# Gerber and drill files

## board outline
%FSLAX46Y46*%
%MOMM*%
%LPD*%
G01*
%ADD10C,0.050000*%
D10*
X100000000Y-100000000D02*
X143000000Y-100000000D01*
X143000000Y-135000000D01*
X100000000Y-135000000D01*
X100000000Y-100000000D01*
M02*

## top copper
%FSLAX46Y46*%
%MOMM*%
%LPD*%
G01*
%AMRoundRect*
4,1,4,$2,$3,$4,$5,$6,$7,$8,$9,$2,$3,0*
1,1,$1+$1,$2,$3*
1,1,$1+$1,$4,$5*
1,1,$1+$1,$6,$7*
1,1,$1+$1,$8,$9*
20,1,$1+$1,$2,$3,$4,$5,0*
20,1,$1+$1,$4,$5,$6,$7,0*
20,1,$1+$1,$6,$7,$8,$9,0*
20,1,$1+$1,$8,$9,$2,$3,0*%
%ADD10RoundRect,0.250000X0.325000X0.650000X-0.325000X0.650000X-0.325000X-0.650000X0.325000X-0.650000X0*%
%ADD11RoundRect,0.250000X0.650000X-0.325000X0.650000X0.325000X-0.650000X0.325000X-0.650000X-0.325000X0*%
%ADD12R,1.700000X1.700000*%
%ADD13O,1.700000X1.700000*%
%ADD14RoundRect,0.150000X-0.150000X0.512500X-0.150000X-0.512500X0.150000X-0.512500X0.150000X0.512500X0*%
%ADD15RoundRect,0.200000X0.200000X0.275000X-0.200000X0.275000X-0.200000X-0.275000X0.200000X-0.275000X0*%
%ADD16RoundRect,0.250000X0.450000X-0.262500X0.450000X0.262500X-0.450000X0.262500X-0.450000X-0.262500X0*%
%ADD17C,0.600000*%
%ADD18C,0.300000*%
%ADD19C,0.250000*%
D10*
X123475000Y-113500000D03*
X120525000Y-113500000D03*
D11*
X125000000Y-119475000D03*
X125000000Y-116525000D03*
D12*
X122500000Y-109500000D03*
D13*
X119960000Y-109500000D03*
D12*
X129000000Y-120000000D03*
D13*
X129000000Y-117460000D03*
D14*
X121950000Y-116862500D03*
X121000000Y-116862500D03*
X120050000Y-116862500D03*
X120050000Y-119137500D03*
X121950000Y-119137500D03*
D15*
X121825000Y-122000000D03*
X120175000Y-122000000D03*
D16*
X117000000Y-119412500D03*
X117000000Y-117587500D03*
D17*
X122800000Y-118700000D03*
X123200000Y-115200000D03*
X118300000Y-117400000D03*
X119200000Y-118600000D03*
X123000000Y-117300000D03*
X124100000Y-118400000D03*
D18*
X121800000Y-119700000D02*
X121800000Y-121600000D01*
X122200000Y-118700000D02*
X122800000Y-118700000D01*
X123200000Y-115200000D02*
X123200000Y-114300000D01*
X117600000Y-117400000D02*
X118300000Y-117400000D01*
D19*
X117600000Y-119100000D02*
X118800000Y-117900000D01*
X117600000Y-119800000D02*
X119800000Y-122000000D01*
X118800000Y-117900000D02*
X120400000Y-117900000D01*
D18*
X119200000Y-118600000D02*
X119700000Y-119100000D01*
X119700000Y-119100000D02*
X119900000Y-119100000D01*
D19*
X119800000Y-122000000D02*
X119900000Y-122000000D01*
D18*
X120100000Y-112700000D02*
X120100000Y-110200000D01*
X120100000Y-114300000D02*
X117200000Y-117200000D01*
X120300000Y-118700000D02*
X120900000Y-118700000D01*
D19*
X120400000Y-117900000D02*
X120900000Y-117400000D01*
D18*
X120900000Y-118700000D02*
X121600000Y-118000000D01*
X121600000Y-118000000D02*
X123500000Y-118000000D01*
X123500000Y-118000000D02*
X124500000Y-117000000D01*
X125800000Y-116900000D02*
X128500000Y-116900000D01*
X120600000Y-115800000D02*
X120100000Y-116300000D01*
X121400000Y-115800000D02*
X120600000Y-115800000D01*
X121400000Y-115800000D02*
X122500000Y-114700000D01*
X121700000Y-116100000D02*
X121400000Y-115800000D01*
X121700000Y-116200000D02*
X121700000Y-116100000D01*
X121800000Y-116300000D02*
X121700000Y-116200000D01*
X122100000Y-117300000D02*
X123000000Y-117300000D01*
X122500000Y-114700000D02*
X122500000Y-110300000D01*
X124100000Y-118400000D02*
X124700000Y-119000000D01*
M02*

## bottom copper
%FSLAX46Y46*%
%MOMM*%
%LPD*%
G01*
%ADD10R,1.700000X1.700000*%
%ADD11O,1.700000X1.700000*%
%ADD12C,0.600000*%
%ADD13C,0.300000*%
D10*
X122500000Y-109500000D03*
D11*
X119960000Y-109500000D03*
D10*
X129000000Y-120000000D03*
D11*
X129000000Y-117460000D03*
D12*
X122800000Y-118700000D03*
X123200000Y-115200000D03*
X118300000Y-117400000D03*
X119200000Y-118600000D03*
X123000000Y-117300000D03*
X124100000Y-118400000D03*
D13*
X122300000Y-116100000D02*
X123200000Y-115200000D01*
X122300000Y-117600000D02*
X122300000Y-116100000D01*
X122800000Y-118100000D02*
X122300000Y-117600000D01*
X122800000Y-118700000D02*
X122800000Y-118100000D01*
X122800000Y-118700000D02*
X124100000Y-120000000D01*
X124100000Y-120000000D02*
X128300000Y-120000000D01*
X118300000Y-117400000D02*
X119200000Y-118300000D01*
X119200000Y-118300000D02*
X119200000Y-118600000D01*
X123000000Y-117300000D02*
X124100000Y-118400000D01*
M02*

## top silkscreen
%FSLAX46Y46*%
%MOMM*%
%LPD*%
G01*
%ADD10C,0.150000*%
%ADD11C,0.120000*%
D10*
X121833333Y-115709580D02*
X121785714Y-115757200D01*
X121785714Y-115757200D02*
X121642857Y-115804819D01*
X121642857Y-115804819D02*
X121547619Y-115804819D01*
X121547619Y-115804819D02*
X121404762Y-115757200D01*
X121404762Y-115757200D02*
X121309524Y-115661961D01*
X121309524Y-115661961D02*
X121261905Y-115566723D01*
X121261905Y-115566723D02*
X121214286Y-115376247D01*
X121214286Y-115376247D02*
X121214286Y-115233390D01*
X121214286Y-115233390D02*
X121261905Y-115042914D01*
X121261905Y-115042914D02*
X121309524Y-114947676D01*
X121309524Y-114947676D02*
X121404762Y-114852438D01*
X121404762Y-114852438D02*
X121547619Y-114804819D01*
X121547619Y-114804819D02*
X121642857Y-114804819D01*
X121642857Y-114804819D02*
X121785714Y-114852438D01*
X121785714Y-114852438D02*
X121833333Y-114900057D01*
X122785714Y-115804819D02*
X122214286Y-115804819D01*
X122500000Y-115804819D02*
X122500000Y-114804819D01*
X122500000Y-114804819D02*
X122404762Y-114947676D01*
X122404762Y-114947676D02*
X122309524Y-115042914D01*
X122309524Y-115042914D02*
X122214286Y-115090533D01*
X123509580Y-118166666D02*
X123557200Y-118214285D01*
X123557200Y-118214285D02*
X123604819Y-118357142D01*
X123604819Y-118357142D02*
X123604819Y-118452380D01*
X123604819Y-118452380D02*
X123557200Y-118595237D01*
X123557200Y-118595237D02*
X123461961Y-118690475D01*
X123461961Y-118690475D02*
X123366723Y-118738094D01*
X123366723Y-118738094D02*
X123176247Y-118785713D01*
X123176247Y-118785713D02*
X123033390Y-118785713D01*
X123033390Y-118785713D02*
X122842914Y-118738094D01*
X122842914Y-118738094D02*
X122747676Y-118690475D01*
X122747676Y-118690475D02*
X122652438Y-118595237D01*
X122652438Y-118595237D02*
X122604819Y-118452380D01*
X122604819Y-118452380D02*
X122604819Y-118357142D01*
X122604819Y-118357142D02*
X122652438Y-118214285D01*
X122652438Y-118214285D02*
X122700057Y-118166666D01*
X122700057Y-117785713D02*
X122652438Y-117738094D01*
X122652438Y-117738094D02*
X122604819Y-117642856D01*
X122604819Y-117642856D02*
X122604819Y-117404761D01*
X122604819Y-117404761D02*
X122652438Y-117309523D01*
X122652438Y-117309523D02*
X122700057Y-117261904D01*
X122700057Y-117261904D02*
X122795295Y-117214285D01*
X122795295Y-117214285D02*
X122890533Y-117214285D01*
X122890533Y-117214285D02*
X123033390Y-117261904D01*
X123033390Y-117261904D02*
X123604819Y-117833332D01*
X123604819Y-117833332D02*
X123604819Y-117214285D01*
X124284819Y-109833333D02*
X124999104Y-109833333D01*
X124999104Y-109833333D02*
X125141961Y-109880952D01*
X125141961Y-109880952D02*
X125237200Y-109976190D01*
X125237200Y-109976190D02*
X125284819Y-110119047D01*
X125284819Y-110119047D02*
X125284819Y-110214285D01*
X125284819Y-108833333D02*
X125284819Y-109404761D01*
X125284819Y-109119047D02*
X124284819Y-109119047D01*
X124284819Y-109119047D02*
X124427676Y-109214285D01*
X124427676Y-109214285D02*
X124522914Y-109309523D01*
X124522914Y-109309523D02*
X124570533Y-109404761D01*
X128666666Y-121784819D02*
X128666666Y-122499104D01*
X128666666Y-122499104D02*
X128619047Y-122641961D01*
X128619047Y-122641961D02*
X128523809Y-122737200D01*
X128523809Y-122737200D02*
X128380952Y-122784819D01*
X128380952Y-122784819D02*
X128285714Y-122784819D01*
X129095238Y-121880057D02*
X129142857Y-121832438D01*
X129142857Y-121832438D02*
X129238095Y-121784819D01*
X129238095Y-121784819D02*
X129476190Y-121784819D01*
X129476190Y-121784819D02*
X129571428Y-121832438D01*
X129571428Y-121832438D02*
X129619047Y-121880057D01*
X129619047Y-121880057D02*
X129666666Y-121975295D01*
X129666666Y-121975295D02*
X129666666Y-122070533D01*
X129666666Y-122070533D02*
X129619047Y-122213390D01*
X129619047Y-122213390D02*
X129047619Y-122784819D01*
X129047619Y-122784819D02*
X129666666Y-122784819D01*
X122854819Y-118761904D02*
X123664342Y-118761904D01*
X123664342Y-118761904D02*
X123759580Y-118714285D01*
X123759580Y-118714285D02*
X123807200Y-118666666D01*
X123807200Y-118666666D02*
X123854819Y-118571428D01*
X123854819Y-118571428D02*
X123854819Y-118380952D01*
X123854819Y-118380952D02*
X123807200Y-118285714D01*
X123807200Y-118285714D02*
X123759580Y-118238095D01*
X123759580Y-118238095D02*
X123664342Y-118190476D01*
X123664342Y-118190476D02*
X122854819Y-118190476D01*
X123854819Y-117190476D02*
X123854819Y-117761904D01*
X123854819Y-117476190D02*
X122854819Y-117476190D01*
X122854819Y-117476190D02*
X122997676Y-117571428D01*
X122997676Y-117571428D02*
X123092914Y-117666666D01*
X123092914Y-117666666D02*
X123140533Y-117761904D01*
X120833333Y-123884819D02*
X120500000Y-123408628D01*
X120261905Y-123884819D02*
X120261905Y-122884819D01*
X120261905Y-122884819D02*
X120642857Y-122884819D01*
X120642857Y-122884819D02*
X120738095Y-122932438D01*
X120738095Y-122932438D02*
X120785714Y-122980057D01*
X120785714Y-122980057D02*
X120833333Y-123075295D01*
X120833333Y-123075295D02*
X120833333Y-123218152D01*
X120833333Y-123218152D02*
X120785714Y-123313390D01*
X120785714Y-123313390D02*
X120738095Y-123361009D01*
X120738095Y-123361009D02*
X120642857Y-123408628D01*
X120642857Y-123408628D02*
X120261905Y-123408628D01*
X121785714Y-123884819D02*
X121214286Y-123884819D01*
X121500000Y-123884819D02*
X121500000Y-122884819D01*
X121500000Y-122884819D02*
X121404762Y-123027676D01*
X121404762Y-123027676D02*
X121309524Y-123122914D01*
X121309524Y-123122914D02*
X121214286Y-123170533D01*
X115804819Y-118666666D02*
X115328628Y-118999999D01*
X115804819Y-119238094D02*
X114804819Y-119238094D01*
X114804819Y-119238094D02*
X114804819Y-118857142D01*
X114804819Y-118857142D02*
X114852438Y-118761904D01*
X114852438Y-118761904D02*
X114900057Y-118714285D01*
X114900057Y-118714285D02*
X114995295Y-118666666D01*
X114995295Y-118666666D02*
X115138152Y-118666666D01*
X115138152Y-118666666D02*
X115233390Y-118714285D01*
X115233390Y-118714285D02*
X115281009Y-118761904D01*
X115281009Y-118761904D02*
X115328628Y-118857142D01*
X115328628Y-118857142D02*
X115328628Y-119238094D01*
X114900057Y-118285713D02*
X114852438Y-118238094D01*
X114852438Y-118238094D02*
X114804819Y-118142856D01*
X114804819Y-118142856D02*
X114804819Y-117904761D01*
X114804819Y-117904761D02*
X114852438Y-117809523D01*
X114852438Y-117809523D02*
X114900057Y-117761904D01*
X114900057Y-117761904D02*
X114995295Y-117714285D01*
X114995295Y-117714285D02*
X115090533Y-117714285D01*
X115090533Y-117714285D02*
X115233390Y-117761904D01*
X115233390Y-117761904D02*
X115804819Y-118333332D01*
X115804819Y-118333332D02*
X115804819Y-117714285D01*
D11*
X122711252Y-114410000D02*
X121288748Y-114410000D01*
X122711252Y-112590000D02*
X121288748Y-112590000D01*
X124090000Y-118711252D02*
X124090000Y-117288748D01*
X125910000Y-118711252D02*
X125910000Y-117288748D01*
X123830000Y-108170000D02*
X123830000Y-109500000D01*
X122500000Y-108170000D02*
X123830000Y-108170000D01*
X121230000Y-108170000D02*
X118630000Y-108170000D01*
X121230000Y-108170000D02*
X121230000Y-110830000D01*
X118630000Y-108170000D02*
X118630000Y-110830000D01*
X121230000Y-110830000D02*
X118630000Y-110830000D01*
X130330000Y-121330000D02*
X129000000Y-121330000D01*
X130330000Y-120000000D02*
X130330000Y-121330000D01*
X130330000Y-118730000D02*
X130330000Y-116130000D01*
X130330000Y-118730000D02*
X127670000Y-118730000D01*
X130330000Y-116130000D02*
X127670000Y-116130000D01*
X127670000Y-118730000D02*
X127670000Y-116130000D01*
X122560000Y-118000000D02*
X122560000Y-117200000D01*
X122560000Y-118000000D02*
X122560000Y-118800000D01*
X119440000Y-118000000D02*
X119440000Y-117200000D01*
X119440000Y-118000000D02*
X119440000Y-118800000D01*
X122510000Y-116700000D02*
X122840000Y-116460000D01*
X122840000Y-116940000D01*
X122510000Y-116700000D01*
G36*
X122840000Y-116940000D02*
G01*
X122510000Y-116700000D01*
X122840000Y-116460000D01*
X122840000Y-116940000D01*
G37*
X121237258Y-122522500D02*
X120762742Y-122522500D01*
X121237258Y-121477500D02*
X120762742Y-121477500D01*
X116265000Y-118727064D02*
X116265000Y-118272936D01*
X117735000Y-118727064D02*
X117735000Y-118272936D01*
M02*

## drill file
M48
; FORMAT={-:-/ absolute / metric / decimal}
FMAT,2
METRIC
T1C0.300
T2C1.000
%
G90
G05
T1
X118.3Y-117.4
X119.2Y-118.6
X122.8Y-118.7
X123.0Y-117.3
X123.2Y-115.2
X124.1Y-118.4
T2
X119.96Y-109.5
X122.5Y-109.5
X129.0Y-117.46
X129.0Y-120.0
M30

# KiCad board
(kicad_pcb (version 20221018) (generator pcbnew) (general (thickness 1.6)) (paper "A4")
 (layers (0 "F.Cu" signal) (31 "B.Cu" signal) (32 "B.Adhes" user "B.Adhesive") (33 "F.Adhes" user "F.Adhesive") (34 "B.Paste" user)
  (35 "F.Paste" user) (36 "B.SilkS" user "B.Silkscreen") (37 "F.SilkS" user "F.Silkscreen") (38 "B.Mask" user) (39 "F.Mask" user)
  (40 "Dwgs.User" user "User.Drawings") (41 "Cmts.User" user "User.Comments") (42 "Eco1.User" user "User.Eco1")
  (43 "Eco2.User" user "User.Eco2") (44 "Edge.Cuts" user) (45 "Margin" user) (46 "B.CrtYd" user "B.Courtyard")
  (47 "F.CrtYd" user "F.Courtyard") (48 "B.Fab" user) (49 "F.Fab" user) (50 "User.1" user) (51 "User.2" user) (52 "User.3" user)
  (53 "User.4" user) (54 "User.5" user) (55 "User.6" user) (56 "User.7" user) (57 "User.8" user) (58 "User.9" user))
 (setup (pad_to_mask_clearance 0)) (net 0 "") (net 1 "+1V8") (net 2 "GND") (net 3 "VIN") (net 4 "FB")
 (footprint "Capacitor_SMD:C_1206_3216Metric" (layer "F.Cu") (at 122 113.5 180)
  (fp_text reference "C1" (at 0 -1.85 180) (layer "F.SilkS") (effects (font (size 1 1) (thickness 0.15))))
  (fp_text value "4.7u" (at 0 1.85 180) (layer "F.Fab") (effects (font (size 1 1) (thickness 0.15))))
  (fp_line (start -0.711252 -0.91) (end 0.711252 -0.91) (stroke (width 0.12) (type solid)) (layer "F.SilkS"))
  (fp_line (start -0.711252 0.91) (end 0.711252 0.91) (stroke (width 0.12) (type solid)) (layer "F.SilkS"))
  (pad "1" smd roundrect (at -1.475 0 180) (size 1.15 1.8) (layers "F.Cu" "F.Paste" "F.Mask") (roundrect_rratio 0.217391) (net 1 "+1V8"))
  (pad "2" smd roundrect (at 1.475 0 180) (size 1.15 1.8) (layers "F.Cu" "F.Paste" "F.Mask") (roundrect_rratio 0.217391) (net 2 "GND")))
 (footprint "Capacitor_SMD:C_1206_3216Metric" (layer "F.Cu") (at 125 118 90)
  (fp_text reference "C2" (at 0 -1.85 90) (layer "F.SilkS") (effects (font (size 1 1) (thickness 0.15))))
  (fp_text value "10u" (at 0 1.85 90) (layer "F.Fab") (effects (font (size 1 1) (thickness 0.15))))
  (fp_line (start -0.711252 -0.91) (end 0.711252 -0.91) (stroke (width 0.12) (type solid)) (layer "F.SilkS"))
  (fp_line (start -0.711252 0.91) (end 0.711252 0.91) (stroke (width 0.12) (type solid)) (layer "F.SilkS"))
  (pad "1" smd roundrect (at -1.475 0 90) (size 1.15 1.8) (layers "F.Cu" "F.Paste" "F.Mask") (roundrect_rratio 0.217391) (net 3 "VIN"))
  (pad "2" smd roundrect (at 1.475 0 90) (size 1.15 1.8) (layers "F.Cu" "F.Paste" "F.Mask") (roundrect_rratio 0.217391) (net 2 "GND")))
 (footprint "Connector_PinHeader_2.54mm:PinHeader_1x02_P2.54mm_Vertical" (layer "F.Cu") (at 122.5 109.5 -90)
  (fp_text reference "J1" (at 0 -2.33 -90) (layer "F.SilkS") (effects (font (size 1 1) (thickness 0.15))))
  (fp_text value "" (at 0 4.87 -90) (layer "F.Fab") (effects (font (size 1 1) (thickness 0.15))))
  (fp_line (start -1.33 -1.33) (end 0 -1.33) (stroke (width 0.12) (type solid)) (layer "F.SilkS"))
  (fp_line (start -1.33 0) (end -1.33 -1.33) (stroke (width 0.12) (type solid)) (layer "F.SilkS"))
  (fp_line (start -1.33 1.27) (end -1.33 3.87) (stroke (width 0.12) (type solid)) (layer "F.SilkS"))
  (fp_line (start -1.33 1.27) (end 1.33 1.27) (stroke (width 0.12) (type solid)) (layer "F.SilkS"))
  (fp_line (start -1.33 3.87) (end 1.33 3.87) (stroke (width 0.12) (type solid)) (layer "F.SilkS"))
  (fp_line (start 1.33 1.27) (end 1.33 3.87) (stroke (width 0.12) (type solid)) (layer "F.SilkS"))
  (pad "1" thru_hole rect (at 0 0 270) (size 1.7 1.7) (drill 1) (layers "*.Cu" "*.Mask") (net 3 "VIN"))
  (pad "2" thru_hole oval (at 0 2.54 270) (size 1.7 1.7) (drill 1) (layers "*.Cu" "*.Mask") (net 2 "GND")))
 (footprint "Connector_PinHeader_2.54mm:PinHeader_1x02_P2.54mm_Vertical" (layer "F.Cu") (at 129 120 180)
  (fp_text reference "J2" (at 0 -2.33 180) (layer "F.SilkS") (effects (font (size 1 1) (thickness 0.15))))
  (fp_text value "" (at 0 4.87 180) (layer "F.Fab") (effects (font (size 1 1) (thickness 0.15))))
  (fp_line (start -1.33 -1.33) (end 0 -1.33) (stroke (width 0.12) (type solid)) (layer "F.SilkS"))
  (fp_line (start -1.33 0) (end -1.33 -1.33) (stroke (width 0.12) (type solid)) (layer "F.SilkS"))
  (fp_line (start -1.33 1.27) (end -1.33 3.87) (stroke (width 0.12) (type solid)) (layer "F.SilkS"))
  (fp_line (start -1.33 1.27) (end 1.33 1.27) (stroke (width 0.12) (type solid)) (layer "F.SilkS"))
  (fp_line (start -1.33 3.87) (end 1.33 3.87) (stroke (width 0.12) (type solid)) (layer "F.SilkS"))
  (fp_line (start 1.33 1.27) (end 1.33 3.87) (stroke (width 0.12) (type solid)) (layer "F.SilkS"))
  (pad "1" thru_hole rect (at 0 0 180) (size 1.7 1.7) (drill 1) (layers "*.Cu" "*.Mask") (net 1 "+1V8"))
  (pad "2" thru_hole oval (at 0 2.54 180) (size 1.7 1.7) (drill 1) (layers "*.Cu" "*.Mask") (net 2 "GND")))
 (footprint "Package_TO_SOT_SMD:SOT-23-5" (layer "F.Cu") (at 121 118 -90)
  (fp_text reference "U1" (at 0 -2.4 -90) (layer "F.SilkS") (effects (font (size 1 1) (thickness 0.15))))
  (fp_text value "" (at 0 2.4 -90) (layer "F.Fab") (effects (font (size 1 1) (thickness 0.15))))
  (fp_line (start 0 -1.56) (end -0.8 -1.56) (stroke (width 0.12) (type solid)) (layer "F.SilkS"))
  (fp_line (start 0 -1.56) (end 0.8 -1.56) (stroke (width 0.12) (type solid)) (layer "F.SilkS"))
  (fp_line (start 0 1.56) (end -0.8 1.56) (stroke (width 0.12) (type solid)) (layer "F.SilkS"))
  (fp_line (start 0 1.56) (end 0.8 1.56) (stroke (width 0.12) (type solid)) (layer "F.SilkS"))
  (fp_poly
   (pts (xy -1.3 -1.51) (xy -1.54 -1.84) (xy -1.06 -1.84) (xy -1.3 -1.51)) (stroke (width 0.12) (type solid)) (fill solid) (layer "F.SilkS"))
  (pad "1" smd roundrect (at -1.1375 -0.95 270) (size 1.325 0.6) (layers "F.Cu" "F.Paste" "F.Mask") (roundrect_rratio 0.25) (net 3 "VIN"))
  (pad "2" smd roundrect (at -1.1375 0 270) (size 1.325 0.6) (layers "F.Cu" "F.Paste" "F.Mask") (roundrect_rratio 0.25) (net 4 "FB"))
  (pad "3" smd roundrect (at -1.1375 0.95 270) (size 1.325 0.6) (layers "F.Cu" "F.Paste" "F.Mask") (roundrect_rratio 0.25) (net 3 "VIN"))
  (pad "4" smd roundrect (at 1.1375 0.95 270) (size 1.325 0.6) (layers "F.Cu" "F.Paste" "F.Mask") (roundrect_rratio 0.25) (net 2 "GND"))
  (pad "5" smd roundrect (at 1.1375 -0.95 270) (size 1.325 0.6) (layers "F.Cu" "F.Paste" "F.Mask") (roundrect_rratio 0.25) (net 1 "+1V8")))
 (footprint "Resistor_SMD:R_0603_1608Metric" (layer "F.Cu") (at 121 122 180)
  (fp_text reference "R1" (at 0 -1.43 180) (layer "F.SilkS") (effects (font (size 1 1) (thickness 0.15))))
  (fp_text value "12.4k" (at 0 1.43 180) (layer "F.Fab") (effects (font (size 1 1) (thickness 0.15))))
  (fp_line (start -0.237258 -0.5225) (end 0.237258 -0.5225) (stroke (width 0.12) (type solid)) (layer "F.SilkS"))
  (fp_line (start -0.237258 0.5225) (end 0.237258 0.5225) (stroke (width 0.12) (type solid)) (layer "F.SilkS"))
  (pad "1" smd roundrect (at -0.825 0 180) (size 0.8 0.95) (layers "F.Cu" "F.Paste" "F.Mask") (roundrect_rratio 0.25) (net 1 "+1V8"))
  (pad "2" smd roundrect (at 0.825 0 180) (size 0.8 0.95) (layers "F.Cu" "F.Paste" "F.Mask") (roundrect_rratio 0.25) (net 4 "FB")))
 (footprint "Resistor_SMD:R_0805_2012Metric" (layer "F.Cu") (at 117 118.5 90)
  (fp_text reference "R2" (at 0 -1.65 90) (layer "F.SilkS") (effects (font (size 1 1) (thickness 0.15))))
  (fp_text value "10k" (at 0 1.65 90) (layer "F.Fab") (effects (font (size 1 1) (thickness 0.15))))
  (fp_line (start -0.227064 -0.735) (end 0.227064 -0.735) (stroke (width 0.12) (type solid)) (layer "F.SilkS"))
  (fp_line (start -0.227064 0.735) (end 0.227064 0.735) (stroke (width 0.12) (type solid)) (layer "F.SilkS"))
  (pad "1" smd roundrect (at -0.9125 0 90) (size 1.025 1.4) (layers "F.Cu" "F.Paste" "F.Mask") (roundrect_rratio 0.243902) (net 4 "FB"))
  (pad "2" smd roundrect (at 0.9125 0 90) (size 1.025 1.4) (layers "F.Cu" "F.Paste" "F.Mask") (roundrect_rratio 0.243902) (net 2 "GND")))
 (gr_rect (start 100 100) (end 143 135) (stroke (width 0.05) (type default)) (fill none) (layer "Edge.Cuts"))
 (segment (start 121.8 119.7) (end 121.8 121.6) (width 0.3) (layer "F.Cu") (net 1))
 (segment (start 122.2 118.7) (end 122.8 118.7) (width 0.3) (layer "F.Cu") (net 1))
 (segment (start 123.2 115.2) (end 123.2 114.3) (width 0.3) (layer "F.Cu") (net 1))
 (via (at 122.8 118.7) (size 0.6) (drill 0.3) (layers "F.Cu" "B.Cu") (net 1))
 (via (at 123.2 115.2) (size 0.6) (drill 0.3) (layers "F.Cu" "B.Cu") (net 1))
 (segment (start 117.6 117.4) (end 118.3 117.4) (width 0.3) (layer "F.Cu") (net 2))
 (segment (start 117.6 119.1) (end 118.8 117.9) (width 0.25) (layer "F.Cu") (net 4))
 (segment (start 117.6 119.8) (end 119.8 122) (width 0.25) (layer "F.Cu") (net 4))
 (segment (start 118.8 117.9) (end 120.4 117.9) (width 0.25) (layer "F.Cu") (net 4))
 (segment (start 119.2 118.6) (end 119.7 119.1) (width 0.3) (layer "F.Cu") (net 2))
 (segment (start 119.7 119.1) (end 119.9 119.1) (width 0.3) (layer "F.Cu") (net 2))
 (segment (start 119.8 122) (end 119.9 122) (width 0.25) (layer "F.Cu") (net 4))
 (segment (start 120.1 112.7) (end 120.1 110.2) (width 0.3) (layer "F.Cu") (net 2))
 (segment (start 120.1 114.3) (end 117.2 117.2) (width 0.3) (layer "F.Cu") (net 2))
 (segment (start 120.3 118.7) (end 120.9 118.7) (width 0.3) (layer "F.Cu") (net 2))
 (segment (start 120.4 117.9) (end 120.9 117.4) (width 0.25) (layer "F.Cu") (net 4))
 (segment (start 120.9 118.7) (end 121.6 118) (width 0.3) (layer "F.Cu") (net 2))
 (segment (start 121.6 118) (end 123.5 118) (width 0.3) (layer "F.Cu") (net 2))
 (segment (start 122.3 116.1) (end 123.2 115.2) (width 0.3) (layer "B.Cu") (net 1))
 (segment (start 122.3 117.6) (end 122.3 116.1) (width 0.3) (layer "B.Cu") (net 1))
 (segment (start 122.8 118.1) (end 122.3 117.6) (width 0.3) (layer "B.Cu") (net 1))
 (segment (start 122.8 118.7) (end 122.8 118.1) (width 0.3) (layer "B.Cu") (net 1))
 (segment (start 122.8 118.7) (end 124.1 120) (width 0.3) (layer "B.Cu") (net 1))
 (segment (start 123.5 118) (end 124.5 117) (width 0.3) (layer "F.Cu") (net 2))
 (segment (start 124.1 120) (end 128.3 120) (width 0.3) (layer "B.Cu") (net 1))
 (segment (start 125.8 116.9) (end 128.5 116.9) (width 0.3) (layer "F.Cu") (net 2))
 (via (at 118.3 117.4) (size 0.6) (drill 0.3) (layers "F.Cu" "B.Cu") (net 2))
 (via (at 119.2 118.6) (size 0.6) (drill 0.3) (layers "F.Cu" "B.Cu") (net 2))
 (segment (start 118.3 117.4) (end 119.2 118.3) (width 0.3) (layer "B.Cu") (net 2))
 (segment (start 119.2 118.3) (end 119.2 118.6) (width 0.3) (layer "B.Cu") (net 2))
 (segment (start 120.6 115.8) (end 120.1 116.3) (width 0.3) (layer "F.Cu") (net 3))
 (segment (start 121.4 115.8) (end 120.6 115.8) (width 0.3) (layer "F.Cu") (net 3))
 (segment (start 121.4 115.8) (end 122.5 114.7) (width 0.3) (layer "F.Cu") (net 3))
 (segment (start 121.7 116.1) (end 121.4 115.8) (width 0.3) (layer "F.Cu") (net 3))
 (segment (start 121.7 116.2) (end 121.7 116.1) (width 0.3) (layer "F.Cu") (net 3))
 (segment (start 121.8 116.3) (end 121.7 116.2) (width 0.3) (layer "F.Cu") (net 3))
 (segment (start 122.1 117.3) (end 123 117.3) (width 0.3) (layer "F.Cu") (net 3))
 (segment (start 122.5 114.7) (end 122.5 110.3) (width 0.3) (layer "F.Cu") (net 3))
 (segment (start 124.1 118.4) (end 124.7 119) (width 0.3) (layer "F.Cu") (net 3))
 (via (at 123 117.3) (size 0.6) (drill 0.3) (layers "F.Cu" "B.Cu") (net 3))
 (via (at 124.1 118.4) (size 0.6) (drill 0.3) (layers "F.Cu" "B.Cu") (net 3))
 (segment (start 123 117.3) (end 124.1 118.4) (width 0.3) (layer "B.Cu") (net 3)))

